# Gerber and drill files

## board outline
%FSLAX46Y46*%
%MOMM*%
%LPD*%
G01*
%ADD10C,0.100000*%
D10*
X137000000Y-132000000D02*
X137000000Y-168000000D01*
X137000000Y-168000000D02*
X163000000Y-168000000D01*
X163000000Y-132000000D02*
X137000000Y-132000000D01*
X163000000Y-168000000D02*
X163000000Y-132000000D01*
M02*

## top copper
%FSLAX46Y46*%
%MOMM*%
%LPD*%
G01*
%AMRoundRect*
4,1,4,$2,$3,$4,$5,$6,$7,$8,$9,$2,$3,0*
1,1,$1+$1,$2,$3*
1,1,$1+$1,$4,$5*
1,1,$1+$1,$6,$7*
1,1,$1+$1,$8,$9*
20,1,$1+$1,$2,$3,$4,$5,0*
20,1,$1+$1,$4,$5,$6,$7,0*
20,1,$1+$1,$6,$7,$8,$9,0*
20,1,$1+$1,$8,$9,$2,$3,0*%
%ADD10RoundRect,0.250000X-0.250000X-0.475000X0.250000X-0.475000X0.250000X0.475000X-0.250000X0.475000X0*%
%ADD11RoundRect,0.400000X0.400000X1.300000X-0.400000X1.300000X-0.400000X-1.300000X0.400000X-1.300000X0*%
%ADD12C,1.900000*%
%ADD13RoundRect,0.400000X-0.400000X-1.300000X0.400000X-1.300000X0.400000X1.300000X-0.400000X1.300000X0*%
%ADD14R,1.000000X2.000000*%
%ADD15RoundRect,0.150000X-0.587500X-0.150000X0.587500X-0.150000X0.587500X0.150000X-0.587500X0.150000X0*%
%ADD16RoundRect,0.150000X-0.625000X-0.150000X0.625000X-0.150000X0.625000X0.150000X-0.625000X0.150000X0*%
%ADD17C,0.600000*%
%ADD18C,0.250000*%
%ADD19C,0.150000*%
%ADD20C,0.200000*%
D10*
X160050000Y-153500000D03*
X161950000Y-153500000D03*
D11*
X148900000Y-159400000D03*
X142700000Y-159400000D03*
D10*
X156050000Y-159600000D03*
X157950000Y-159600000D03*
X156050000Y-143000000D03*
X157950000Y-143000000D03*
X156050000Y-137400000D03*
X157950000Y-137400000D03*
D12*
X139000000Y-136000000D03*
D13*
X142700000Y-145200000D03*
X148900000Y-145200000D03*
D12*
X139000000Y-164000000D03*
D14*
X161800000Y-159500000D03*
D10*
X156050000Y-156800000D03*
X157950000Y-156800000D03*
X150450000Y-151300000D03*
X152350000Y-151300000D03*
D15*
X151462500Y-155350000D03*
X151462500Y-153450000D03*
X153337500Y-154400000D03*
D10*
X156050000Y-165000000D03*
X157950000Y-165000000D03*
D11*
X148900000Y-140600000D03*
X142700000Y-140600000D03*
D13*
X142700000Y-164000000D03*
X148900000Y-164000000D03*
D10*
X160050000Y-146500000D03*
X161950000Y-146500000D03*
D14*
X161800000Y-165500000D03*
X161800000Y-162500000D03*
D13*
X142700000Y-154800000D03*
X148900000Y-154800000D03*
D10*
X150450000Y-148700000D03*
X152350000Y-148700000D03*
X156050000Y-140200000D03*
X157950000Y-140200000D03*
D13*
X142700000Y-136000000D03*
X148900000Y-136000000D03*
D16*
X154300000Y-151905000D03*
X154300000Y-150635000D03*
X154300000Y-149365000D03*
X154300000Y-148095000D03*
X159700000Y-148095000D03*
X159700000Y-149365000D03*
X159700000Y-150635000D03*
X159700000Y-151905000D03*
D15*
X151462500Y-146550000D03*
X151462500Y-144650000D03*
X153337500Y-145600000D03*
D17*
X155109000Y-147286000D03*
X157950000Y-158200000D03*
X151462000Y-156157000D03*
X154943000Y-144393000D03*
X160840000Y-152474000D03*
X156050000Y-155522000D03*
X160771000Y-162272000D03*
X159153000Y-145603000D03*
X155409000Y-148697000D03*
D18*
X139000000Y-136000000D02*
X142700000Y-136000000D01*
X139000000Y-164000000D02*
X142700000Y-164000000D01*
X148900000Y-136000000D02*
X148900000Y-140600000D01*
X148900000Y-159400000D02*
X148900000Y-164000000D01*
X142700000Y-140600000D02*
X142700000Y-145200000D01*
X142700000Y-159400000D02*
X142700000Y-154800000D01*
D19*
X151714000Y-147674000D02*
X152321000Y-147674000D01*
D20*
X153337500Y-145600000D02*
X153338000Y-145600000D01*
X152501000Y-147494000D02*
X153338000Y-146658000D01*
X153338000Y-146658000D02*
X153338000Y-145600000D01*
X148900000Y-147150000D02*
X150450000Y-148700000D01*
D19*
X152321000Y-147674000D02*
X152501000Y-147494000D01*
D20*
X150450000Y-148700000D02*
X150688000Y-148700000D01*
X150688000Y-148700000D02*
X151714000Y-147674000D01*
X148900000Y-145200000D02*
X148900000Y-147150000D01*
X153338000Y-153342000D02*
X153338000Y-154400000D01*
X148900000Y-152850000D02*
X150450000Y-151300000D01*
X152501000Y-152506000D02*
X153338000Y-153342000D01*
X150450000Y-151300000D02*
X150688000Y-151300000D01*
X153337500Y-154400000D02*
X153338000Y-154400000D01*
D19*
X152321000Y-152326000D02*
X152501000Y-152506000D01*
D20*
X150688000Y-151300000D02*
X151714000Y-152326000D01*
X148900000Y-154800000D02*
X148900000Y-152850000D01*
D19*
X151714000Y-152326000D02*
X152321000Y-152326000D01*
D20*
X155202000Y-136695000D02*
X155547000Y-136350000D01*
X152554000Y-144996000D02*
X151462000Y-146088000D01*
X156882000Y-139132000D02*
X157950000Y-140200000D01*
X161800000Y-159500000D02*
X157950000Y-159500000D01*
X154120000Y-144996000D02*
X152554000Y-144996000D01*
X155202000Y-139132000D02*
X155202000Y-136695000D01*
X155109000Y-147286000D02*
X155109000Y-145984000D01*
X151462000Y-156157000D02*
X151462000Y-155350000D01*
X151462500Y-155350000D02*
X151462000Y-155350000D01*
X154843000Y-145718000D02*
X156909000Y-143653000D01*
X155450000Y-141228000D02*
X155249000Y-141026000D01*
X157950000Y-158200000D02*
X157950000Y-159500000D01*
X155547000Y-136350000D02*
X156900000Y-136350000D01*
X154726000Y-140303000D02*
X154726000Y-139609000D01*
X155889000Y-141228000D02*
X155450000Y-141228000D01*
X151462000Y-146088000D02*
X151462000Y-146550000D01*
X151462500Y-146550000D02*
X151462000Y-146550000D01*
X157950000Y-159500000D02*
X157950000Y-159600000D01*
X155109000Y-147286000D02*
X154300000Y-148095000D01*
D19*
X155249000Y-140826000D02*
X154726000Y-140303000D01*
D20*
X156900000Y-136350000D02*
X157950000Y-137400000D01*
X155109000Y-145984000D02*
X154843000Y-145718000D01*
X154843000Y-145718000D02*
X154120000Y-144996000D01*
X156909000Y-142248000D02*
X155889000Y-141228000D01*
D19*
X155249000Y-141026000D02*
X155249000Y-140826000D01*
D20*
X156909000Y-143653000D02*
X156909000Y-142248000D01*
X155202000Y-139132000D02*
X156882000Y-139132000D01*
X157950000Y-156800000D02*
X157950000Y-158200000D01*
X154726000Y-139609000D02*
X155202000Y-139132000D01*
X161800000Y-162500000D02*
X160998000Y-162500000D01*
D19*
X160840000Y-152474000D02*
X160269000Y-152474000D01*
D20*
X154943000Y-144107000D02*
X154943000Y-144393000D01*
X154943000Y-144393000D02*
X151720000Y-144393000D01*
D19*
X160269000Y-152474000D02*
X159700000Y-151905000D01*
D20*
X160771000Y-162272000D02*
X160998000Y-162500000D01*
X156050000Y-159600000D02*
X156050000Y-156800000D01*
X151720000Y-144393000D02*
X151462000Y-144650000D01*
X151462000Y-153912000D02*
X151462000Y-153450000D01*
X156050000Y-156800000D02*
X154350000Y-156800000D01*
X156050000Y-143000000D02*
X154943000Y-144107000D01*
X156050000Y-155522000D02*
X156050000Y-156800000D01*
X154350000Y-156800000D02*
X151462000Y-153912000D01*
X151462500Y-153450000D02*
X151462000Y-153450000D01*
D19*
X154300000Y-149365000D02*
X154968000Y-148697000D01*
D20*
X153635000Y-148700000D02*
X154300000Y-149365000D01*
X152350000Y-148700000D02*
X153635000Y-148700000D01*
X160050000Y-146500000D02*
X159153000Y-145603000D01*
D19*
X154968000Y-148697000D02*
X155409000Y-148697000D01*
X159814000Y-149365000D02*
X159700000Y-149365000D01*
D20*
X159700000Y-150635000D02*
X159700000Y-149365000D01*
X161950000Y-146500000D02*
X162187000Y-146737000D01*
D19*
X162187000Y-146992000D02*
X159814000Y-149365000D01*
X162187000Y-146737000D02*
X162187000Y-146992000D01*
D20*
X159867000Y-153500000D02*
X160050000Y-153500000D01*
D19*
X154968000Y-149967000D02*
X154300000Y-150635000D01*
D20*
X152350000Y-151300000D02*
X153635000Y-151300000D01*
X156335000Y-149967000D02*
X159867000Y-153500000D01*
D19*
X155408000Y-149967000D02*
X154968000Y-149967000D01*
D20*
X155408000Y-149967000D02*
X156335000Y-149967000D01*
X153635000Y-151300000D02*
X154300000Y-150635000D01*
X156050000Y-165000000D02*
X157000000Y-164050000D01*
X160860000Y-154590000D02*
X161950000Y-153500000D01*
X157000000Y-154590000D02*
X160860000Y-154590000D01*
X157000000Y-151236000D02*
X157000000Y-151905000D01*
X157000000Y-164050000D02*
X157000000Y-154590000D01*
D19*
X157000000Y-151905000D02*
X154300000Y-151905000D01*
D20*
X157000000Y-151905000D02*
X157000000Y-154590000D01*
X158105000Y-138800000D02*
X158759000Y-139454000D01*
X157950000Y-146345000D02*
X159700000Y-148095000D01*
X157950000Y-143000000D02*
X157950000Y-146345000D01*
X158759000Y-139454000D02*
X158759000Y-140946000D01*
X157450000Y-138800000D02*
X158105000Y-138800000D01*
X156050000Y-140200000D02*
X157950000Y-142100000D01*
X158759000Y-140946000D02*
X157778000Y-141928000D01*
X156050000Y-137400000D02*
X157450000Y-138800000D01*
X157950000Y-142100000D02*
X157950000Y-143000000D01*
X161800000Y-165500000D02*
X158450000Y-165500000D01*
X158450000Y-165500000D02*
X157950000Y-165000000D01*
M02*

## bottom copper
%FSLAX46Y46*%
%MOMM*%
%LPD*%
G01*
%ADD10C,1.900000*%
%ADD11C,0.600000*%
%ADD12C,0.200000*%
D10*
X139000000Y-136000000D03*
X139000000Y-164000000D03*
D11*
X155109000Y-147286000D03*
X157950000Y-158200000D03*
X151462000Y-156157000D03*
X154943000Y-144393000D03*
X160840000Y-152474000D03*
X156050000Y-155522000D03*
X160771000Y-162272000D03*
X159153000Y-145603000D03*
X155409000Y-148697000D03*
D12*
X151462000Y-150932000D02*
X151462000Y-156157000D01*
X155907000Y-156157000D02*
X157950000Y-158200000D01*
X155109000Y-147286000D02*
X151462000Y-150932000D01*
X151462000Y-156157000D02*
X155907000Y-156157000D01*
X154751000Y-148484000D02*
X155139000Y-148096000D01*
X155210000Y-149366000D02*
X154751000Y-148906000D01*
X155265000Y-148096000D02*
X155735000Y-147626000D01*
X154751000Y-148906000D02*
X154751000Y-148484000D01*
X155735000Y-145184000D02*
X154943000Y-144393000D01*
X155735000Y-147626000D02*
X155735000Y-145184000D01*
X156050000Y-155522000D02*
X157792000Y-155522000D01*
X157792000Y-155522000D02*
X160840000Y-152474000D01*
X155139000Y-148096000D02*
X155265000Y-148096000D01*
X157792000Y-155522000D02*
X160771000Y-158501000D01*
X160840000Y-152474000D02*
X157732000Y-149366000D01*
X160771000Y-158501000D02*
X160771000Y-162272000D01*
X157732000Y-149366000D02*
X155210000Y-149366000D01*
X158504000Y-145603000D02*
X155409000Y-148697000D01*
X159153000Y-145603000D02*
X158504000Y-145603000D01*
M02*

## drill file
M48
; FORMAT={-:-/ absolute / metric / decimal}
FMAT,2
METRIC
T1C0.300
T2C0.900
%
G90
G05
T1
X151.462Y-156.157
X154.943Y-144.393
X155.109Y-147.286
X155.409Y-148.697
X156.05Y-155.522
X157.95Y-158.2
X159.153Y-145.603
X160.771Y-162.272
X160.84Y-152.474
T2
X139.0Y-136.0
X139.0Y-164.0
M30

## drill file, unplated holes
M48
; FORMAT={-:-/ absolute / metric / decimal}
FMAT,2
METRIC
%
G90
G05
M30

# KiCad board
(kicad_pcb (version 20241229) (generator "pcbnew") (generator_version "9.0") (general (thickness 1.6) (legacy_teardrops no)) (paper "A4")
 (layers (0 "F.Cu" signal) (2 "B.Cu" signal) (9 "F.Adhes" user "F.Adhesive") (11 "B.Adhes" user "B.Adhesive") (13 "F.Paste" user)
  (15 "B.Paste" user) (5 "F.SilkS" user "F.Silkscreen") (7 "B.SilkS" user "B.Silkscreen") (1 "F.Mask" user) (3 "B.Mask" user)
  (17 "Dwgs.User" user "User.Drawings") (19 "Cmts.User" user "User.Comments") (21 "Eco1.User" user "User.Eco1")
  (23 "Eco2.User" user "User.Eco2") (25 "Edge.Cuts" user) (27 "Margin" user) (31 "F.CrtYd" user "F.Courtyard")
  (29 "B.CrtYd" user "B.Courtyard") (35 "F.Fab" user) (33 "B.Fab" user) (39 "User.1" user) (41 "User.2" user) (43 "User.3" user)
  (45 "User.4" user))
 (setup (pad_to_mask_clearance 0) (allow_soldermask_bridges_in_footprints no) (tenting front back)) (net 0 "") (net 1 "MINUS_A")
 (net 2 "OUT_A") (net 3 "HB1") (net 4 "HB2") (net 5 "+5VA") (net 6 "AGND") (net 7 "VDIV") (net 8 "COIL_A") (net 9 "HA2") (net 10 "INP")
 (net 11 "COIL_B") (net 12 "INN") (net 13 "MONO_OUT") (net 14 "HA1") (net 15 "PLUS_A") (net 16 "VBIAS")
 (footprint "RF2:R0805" (layer "F.Cu") (at 161 153.5)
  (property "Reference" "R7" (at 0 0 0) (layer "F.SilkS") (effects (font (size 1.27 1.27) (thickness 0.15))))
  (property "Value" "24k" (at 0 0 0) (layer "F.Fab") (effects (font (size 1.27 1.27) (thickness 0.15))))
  (pad "1" smd roundrect (at -0.95 0) (size 1 1.45) (layers "F.Cu" "F.Mask" "F.Paste") (roundrect_rratio 0.25) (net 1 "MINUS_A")
   (thermal_bridge_angle 45))
  (pad "2" smd roundrect (at 0.95 0) (size 1 1.45) (layers "F.Cu" "F.Mask" "F.Paste") (roundrect_rratio 0.25) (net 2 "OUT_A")
   (thermal_bridge_angle 45)))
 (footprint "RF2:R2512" (layer "F.Cu") (at 145.8 159.4 180)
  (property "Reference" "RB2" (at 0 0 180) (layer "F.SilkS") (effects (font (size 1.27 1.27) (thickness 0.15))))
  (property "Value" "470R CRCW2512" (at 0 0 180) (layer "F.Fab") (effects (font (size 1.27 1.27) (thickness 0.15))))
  (pad "1" smd roundrect (at -3.1 0 180) (size 1.6 3.4) (layers "F.Cu" "F.Mask" "F.Paste") (roundrect_rratio 0.25) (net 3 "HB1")
   (thermal_bridge_angle 45))
  (pad "2" smd roundrect (at 3.1 0 180) (size 1.6 3.4) (layers "F.Cu" "F.Mask" "F.Paste") (roundrect_rratio 0.25) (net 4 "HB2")
   (thermal_bridge_angle 45)))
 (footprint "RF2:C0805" (layer "F.Cu") (at 157 159.6)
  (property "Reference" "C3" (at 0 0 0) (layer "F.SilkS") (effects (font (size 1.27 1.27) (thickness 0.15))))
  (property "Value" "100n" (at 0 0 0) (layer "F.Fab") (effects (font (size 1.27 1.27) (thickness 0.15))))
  (pad "1" smd roundrect (at -0.95 0) (size 1 1.45) (layers "F.Cu" "F.Mask" "F.Paste") (roundrect_rratio 0.25) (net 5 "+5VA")
   (thermal_bridge_angle 45))
  (pad "2" smd roundrect (at 0.95 0) (size 1 1.45) (layers "F.Cu" "F.Mask" "F.Paste") (roundrect_rratio 0.25) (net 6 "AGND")
   (thermal_bridge_angle 45)))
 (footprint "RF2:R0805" (layer "F.Cu") (at 157 143)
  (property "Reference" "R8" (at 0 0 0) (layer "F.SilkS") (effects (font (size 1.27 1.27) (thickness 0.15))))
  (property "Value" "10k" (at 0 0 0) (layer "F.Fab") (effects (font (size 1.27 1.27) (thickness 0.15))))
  (pad "1" smd roundrect (at -0.95 0) (size 1 1.45) (layers "F.Cu" "F.Mask" "F.Paste") (roundrect_rratio 0.25) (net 5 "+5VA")
   (thermal_bridge_angle 45))
  (pad "2" smd roundrect (at 0.95 0) (size 1 1.45) (layers "F.Cu" "F.Mask" "F.Paste") (roundrect_rratio 0.25) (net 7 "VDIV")
   (thermal_bridge_angle 45)))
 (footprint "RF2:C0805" (layer "F.Cu") (at 157 137.4)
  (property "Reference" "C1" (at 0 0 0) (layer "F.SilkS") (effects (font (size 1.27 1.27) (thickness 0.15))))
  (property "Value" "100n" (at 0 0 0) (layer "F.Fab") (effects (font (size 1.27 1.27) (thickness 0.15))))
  (pad "1" smd roundrect (at -0.95 0) (size 1 1.45) (layers "F.Cu" "F.Mask" "F.Paste") (roundrect_rratio 0.25) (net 7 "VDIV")
   (thermal_bridge_angle 45))
  (pad "2" smd roundrect (at 0.95 0) (size 1 1.45) (layers "F.Cu" "F.Mask" "F.Paste") (roundrect_rratio 0.25) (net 6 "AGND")
   (thermal_bridge_angle 45)))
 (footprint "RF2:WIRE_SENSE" (layer "F.Cu") (at 139 136)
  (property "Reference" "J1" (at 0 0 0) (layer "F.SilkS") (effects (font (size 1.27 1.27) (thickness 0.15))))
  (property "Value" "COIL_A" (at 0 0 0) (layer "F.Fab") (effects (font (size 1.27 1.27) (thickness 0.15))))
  (pad "1" thru_hole circle (at 0 0) (size 1.9 1.9) (drill 0.9) (layers "*.Cu" "*.Mask") (remove_unused_layers no) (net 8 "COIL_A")))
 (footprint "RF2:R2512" (layer "F.Cu") (at 145.8 145.2)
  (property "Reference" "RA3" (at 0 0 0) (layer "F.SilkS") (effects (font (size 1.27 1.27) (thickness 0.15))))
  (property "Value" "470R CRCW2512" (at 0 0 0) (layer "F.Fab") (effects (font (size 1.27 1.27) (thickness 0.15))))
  (pad "1" smd roundrect (at -3.1 0) (size 1.6 3.4) (layers "F.Cu" "F.Mask" "F.Paste") (roundrect_rratio 0.25) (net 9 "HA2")
   (thermal_bridge_angle 45))
  (pad "2" smd roundrect (at 3.1 0) (size 1.6 3.4) (layers "F.Cu" "F.Mask" "F.Paste") (roundrect_rratio 0.25) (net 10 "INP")
   (thermal_bridge_angle 45)))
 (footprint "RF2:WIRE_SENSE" (layer "F.Cu") (at 139 164)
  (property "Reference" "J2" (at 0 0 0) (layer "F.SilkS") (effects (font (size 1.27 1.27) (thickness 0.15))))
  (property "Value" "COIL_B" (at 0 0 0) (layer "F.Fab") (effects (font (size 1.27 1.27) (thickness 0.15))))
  (pad "1" thru_hole circle (at 0 0) (size 1.9 1.9) (drill 0.9) (layers "*.Cu" "*.Mask") (remove_unused_layers no) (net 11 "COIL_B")))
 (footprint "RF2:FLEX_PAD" (layer "F.Cu") (at 161.8 159.5)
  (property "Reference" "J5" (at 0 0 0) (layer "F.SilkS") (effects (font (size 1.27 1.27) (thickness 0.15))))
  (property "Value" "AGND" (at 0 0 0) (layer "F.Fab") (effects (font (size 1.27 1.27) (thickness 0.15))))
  (pad "1" smd rect (at 0 0) (size 1 2) (layers "F.Cu" "F.Mask" "F.Paste") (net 6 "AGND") (thermal_bridge_angle 45)))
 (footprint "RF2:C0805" (layer "F.Cu") (at 157 156.8)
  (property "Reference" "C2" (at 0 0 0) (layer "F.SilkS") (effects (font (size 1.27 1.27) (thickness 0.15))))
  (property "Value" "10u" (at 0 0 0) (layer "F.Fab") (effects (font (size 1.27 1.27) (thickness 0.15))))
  (pad "1" smd roundrect (at -0.95 0) (size 1 1.45) (layers "F.Cu" "F.Mask" "F.Paste") (roundrect_rratio 0.25) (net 5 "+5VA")
   (thermal_bridge_angle 45))
  (pad "2" smd roundrect (at 0.95 0) (size 1 1.45) (layers "F.Cu" "F.Mask" "F.Paste") (roundrect_rratio 0.25) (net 6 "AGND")
   (thermal_bridge_angle 45)))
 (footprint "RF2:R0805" (layer "F.Cu") (at 151.4 151.3)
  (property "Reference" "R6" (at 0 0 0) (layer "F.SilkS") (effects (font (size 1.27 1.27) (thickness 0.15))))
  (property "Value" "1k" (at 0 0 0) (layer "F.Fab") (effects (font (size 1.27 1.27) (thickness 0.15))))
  (pad "1" smd roundrect (at -0.95 0) (size 1 1.45) (layers "F.Cu" "F.Mask" "F.Paste") (roundrect_rratio 0.25) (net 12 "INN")
   (thermal_bridge_angle 45))
  (pad "2" smd roundrect (at 0.95 0) (size 1 1.45) (layers "F.Cu" "F.Mask" "F.Paste") (roundrect_rratio 0.25) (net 1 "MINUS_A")
   (thermal_bridge_angle 45)))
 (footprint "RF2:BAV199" (layer "F.Cu") (at 152.4 154.4)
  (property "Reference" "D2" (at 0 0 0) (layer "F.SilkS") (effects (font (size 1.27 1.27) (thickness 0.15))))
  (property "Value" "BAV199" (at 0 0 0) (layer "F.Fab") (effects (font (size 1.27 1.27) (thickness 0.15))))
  (pad "1" smd roundrect (at -0.9375 0.95) (size 1.475 0.6) (layers "F.Cu" "F.Mask" "F.Paste") (roundrect_rratio 0.25) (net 6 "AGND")
   (thermal_bridge_angle 45))
  (pad "2" smd roundrect (at -0.9375 -0.95) (size 1.475 0.6) (layers "F.Cu" "F.Mask" "F.Paste") (roundrect_rratio 0.25) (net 5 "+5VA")
   (thermal_bridge_angle 45))
  (pad "3" smd roundrect (at 0.9375 0) (size 1.475 0.6) (layers "F.Cu" "F.Mask" "F.Paste") (roundrect_rratio 0.25) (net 12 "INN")
   (thermal_bridge_angle 45)))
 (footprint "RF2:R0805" (layer "F.Cu") (at 157 165)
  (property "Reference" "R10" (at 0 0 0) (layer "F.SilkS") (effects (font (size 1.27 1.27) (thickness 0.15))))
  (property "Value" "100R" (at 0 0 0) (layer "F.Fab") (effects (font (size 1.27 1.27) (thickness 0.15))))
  (pad "1" smd roundrect (at -0.95 0) (size 1 1.45) (layers "F.Cu" "F.Mask" "F.Paste") (roundrect_rratio 0.25) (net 2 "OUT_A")
   (thermal_bridge_angle 45))
  (pad "2" smd roundrect (at 0.95 0) (size 1 1.45) (layers "F.Cu" "F.Mask" "F.Paste") (roundrect_rratio 0.25) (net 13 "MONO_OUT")
   (thermal_bridge_angle 45)))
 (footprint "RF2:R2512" (layer "F.Cu") (at 145.8 140.6 180)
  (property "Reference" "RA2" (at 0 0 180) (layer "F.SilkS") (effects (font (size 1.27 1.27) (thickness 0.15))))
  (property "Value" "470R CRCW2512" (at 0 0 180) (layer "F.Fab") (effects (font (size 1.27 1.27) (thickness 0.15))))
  (pad "1" smd roundrect (at -3.1 0 180) (size 1.6 3.4) (layers "F.Cu" "F.Mask" "F.Paste") (roundrect_rratio 0.25) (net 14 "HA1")
   (thermal_bridge_angle 45))
  (pad "2" smd roundrect (at 3.1 0 180) (size 1.6 3.4) (layers "F.Cu" "F.Mask" "F.Paste") (roundrect_rratio 0.25) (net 9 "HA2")
   (thermal_bridge_angle 45)))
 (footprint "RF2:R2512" (layer "F.Cu") (at 145.8 164)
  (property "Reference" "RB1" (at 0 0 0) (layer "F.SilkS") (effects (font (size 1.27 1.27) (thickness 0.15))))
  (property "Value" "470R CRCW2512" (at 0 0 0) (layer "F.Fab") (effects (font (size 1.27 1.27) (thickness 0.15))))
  (pad "1" smd roundrect (at -3.1 0) (size 1.6 3.4) (layers "F.Cu" "F.Mask" "F.Paste") (roundrect_rratio 0.25) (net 11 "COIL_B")
   (thermal_bridge_angle 45))
  (pad "2" smd roundrect (at 3.1 0) (size 1.6 3.4) (layers "F.Cu" "F.Mask" "F.Paste") (roundrect_rratio 0.25) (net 3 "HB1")
   (thermal_bridge_angle 45)))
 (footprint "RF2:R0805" (layer "F.Cu") (at 161 146.5)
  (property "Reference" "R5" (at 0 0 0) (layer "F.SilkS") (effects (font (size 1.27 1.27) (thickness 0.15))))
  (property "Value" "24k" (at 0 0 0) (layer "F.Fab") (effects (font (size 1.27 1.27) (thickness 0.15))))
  (pad "1" smd roundrect (at -0.95 0) (size 1 1.45) (layers "F.Cu" "F.Mask" "F.Paste") (roundrect_rratio 0.25) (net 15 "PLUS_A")
   (thermal_bridge_angle 45))
  (pad "2" smd roundrect (at 0.95 0) (size 1 1.45) (layers "F.Cu" "F.Mask" "F.Paste") (roundrect_rratio 0.25) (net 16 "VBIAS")
   (thermal_bridge_angle 45)))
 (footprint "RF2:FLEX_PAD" (layer "F.Cu") (at 161.8 165.5)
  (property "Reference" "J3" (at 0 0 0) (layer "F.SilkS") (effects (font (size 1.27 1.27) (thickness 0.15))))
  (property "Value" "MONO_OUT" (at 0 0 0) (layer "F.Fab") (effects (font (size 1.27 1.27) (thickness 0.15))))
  (pad "1" smd rect (at 0 0) (size 1 2) (layers "F.Cu" "F.Mask" "F.Paste") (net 13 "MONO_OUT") (thermal_bridge_angle 45)))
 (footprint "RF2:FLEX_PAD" (layer "F.Cu") (at 161.8 162.5)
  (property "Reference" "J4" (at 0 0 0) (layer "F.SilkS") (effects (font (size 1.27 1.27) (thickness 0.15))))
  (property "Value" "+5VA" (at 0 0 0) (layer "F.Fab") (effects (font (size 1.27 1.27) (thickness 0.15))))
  (pad "1" smd rect (at 0 0) (size 1 2) (layers "F.Cu" "F.Mask" "F.Paste") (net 5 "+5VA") (thermal_bridge_angle 45)))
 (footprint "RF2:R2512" (layer "F.Cu") (at 145.8 154.8)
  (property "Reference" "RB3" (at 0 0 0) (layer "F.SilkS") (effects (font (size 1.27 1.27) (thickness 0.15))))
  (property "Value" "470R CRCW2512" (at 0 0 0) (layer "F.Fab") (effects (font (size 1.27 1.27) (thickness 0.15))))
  (pad "1" smd roundrect (at -3.1 0) (size 1.6 3.4) (layers "F.Cu" "F.Mask" "F.Paste") (roundrect_rratio 0.25) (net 4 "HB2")
   (thermal_bridge_angle 45))
  (pad "2" smd roundrect (at 3.1 0) (size 1.6 3.4) (layers "F.Cu" "F.Mask" "F.Paste") (roundrect_rratio 0.25) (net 12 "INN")
   (thermal_bridge_angle 45)))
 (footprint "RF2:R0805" (layer "F.Cu") (at 151.4 148.7)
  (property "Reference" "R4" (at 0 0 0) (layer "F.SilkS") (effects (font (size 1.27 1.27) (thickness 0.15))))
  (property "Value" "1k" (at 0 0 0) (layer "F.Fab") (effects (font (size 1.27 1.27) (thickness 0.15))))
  (pad "1" smd roundrect (at -0.95 0) (size 1 1.45) (layers "F.Cu" "F.Mask" "F.Paste") (roundrect_rratio 0.25) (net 10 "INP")
   (thermal_bridge_angle 45))
  (pad "2" smd roundrect (at 0.95 0) (size 1 1.45) (layers "F.Cu" "F.Mask" "F.Paste") (roundrect_rratio 0.25) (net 15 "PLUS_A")
   (thermal_bridge_angle 45)))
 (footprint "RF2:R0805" (layer "F.Cu") (at 157 140.2)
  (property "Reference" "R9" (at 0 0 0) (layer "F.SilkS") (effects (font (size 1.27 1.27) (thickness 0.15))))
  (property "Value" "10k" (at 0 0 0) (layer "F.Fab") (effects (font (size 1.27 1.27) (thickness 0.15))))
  (pad "1" smd roundrect (at -0.95 0) (size 1 1.45) (layers "F.Cu" "F.Mask" "F.Paste") (roundrect_rratio 0.25) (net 7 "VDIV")
   (thermal_bridge_angle 45))
  (pad "2" smd roundrect (at 0.95 0) (size 1 1.45) (layers "F.Cu" "F.Mask" "F.Paste") (roundrect_rratio 0.25) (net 6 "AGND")
   (thermal_bridge_angle 45)))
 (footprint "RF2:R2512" (layer "F.Cu") (at 145.8 136)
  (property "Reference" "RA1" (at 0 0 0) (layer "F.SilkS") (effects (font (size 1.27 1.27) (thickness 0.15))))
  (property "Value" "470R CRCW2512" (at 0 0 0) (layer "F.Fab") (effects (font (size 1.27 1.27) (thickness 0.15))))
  (pad "1" smd roundrect (at -3.1 0) (size 1.6 3.4) (layers "F.Cu" "F.Mask" "F.Paste") (roundrect_rratio 0.25) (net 8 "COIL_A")
   (thermal_bridge_angle 45))
  (pad "2" smd roundrect (at 3.1 0) (size 1.6 3.4) (layers "F.Cu" "F.Mask" "F.Paste") (roundrect_rratio 0.25) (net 14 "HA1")
   (thermal_bridge_angle 45)))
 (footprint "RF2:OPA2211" (layer "F.Cu") (at 157 150)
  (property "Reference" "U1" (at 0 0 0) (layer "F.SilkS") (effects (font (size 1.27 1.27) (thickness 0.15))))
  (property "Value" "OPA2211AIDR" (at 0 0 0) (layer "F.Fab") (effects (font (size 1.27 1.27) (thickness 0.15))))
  (pad "1" smd roundrect (at -2.7 1.905) (size 1.55 0.6) (layers "F.Cu" "F.Mask" "F.Paste") (roundrect_rratio 0.25) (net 2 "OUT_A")
   (thermal_bridge_angle 45))
  (pad "2" smd roundrect (at -2.7 0.635) (size 1.55 0.6) (layers "F.Cu" "F.Mask" "F.Paste") (roundrect_rratio 0.25) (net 1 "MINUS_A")
   (thermal_bridge_angle 45))
  (pad "3" smd roundrect (at -2.7 -0.635) (size 1.55 0.6) (layers "F.Cu" "F.Mask" "F.Paste") (roundrect_rratio 0.25) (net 15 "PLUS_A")
   (thermal_bridge_angle 45))
  (pad "4" smd roundrect (at -2.7 -1.905) (size 1.55 0.6) (layers "F.Cu" "F.Mask" "F.Paste") (roundrect_rratio 0.25) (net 6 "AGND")
   (thermal_bridge_angle 45))
  (pad "5" smd roundrect (at 2.7 -1.905) (size 1.55 0.6) (layers "F.Cu" "F.Mask" "F.Paste") (roundrect_rratio 0.25) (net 7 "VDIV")
   (thermal_bridge_angle 45))
  (pad "6" smd roundrect (at 2.7 -0.635) (size 1.55 0.6) (layers "F.Cu" "F.Mask" "F.Paste") (roundrect_rratio 0.25) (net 16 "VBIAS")
   (thermal_bridge_angle 45))
  (pad "7" smd roundrect (at 2.7 0.635) (size 1.55 0.6) (layers "F.Cu" "F.Mask" "F.Paste") (roundrect_rratio 0.25) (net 16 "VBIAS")
   (thermal_bridge_angle 45))
  (pad "8" smd roundrect (at 2.7 1.905) (size 1.55 0.6) (layers "F.Cu" "F.Mask" "F.Paste") (roundrect_rratio 0.25) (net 5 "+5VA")
   (thermal_bridge_angle 45)))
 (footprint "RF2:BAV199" (layer "F.Cu") (at 152.4 145.6)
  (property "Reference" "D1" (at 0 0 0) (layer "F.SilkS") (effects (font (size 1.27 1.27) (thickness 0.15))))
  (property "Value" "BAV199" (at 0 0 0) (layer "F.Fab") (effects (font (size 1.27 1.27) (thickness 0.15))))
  (pad "1" smd roundrect (at -0.9375 0.95) (size 1.475 0.6) (layers "F.Cu" "F.Mask" "F.Paste") (roundrect_rratio 0.25) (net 6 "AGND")
   (thermal_bridge_angle 45))
  (pad "2" smd roundrect (at -0.9375 -0.95) (size 1.475 0.6) (layers "F.Cu" "F.Mask" "F.Paste") (roundrect_rratio 0.25) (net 5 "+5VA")
   (thermal_bridge_angle 45))
  (pad "3" smd roundrect (at 0.9375 0) (size 1.475 0.6) (layers "F.Cu" "F.Mask" "F.Paste") (roundrect_rratio 0.25) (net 10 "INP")
   (thermal_bridge_angle 45)))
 (gr_line (start 137 132) (end 137 168) (stroke (width 0.1) (type default)) (layer "Edge.Cuts"))
 (gr_line (start 137 168) (end 163 168) (stroke (width 0.1) (type default)) (layer "Edge.Cuts"))
 (gr_line (start 163 132) (end 137 132) (stroke (width 0.1) (type default)) (layer "Edge.Cuts"))
 (gr_line (start 163 168) (end 163 132) (stroke (width 0.1) (type default)) (layer "Edge.Cuts"))
 (segment (start 139 136) (end 142.7 136) (width 0.25) (layer "F.Cu") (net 8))
 (segment (start 139 164) (end 142.7 164) (width 0.25) (layer "F.Cu") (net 11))
 (segment (start 148.9 136) (end 148.9 140.6) (width 0.25) (layer "F.Cu") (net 14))
 (segment (start 148.9 159.4) (end 148.9 164) (width 0.25) (layer "F.Cu") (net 3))
 (segment (start 142.7 140.6) (end 142.7 145.2) (width 0.25) (layer "F.Cu") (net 9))
 (segment (start 142.7 159.4) (end 142.7 154.8) (width 0.25) (layer "F.Cu") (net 4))
 (segment (start 151.714 147.674) (end 152.321 147.674) (width 0.15) (layer "F.Cu") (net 10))
 (segment (start 153.3375 145.6) (end 153.338 145.6) (width 0.2) (layer "F.Cu") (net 10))
 (segment (start 152.501 147.494) (end 153.338 146.658) (width 0.2) (layer "F.Cu") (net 10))
 (segment (start 153.338 146.658) (end 153.338 145.6) (width 0.2) (layer "F.Cu") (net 10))
 (segment (start 148.9 147.15) (end 150.45 148.7) (width 0.2) (layer "F.Cu") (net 10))
 (segment (start 152.321 147.674) (end 152.501 147.494) (width 0.15) (layer "F.Cu") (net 10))
 (segment (start 150.45 148.7) (end 150.688 148.7) (width 0.2) (layer "F.Cu") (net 10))
 (segment (start 150.688 148.7) (end 151.714 147.674) (width 0.2) (layer "F.Cu") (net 10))
 (segment (start 148.9 145.2) (end 148.9 147.15) (width 0.2) (layer "F.Cu") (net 10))
 (segment (start 153.338 153.342) (end 153.338 154.4) (width 0.2) (layer "F.Cu") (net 12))
 (segment (start 148.9 152.85) (end 150.45 151.3) (width 0.2) (layer "F.Cu") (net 12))
 (segment (start 152.501 152.506) (end 153.338 153.342) (width 0.2) (layer "F.Cu") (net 12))
 (segment (start 150.45 151.3) (end 150.688 151.3) (width 0.2) (layer "F.Cu") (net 12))
 (segment (start 153.3375 154.4) (end 153.338 154.4) (width 0.2) (layer "F.Cu") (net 12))
 (segment (start 152.321 152.326) (end 152.501 152.506) (width 0.15) (layer "F.Cu") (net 12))
 (segment (start 150.688 151.3) (end 151.714 152.326) (width 0.2) (layer "F.Cu") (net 12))
 (segment (start 148.9 154.8) (end 148.9 152.85) (width 0.2) (layer "F.Cu") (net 12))
 (segment (start 151.714 152.326) (end 152.321 152.326) (width 0.15) (layer "F.Cu") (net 12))
 (segment (start 155.202 136.695) (end 155.547 136.35) (width 0.2) (layer "F.Cu") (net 6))
 (segment (start 152.554 144.996) (end 151.462 146.088) (width 0.2) (layer "F.Cu") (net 6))
 (segment (start 156.882 139.132) (end 157.95 140.2) (width 0.2) (layer "F.Cu") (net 6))
 (segment (start 161.8 159.5) (end 157.95 159.5) (width 0.2) (layer "F.Cu") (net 6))
 (segment (start 154.12 144.996) (end 152.554 144.996) (width 0.2) (layer "F.Cu") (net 6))
 (segment (start 155.202 139.132) (end 155.202 136.695) (width 0.2) (layer "F.Cu") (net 6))
 (segment (start 155.109 147.286) (end 155.109 145.984) (width 0.2) (layer "F.Cu") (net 6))
 (segment (start 151.462 156.157) (end 151.462 155.35) (width 0.2) (layer "F.Cu") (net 6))
 (segment (start 151.4625 155.35) (end 151.462 155.35) (width 0.2) (layer "F.Cu") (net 6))
 (segment (start 154.843 145.718) (end 156.909 143.653) (width 0.2) (layer "F.Cu") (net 6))
 (segment (start 155.45 141.228) (end 155.249 141.026) (width 0.2) (layer "F.Cu") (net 6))
 (segment (start 157.95 158.2) (end 157.95 159.5) (width 0.2) (layer "F.Cu") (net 6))
 (segment (start 155.547 136.35) (end 156.9 136.35) (width 0.2) (layer "F.Cu") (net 6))
 (segment (start 154.726 140.303) (end 154.726 139.609) (width 0.2) (layer "F.Cu") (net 6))
 (segment (start 155.889 141.228) (end 155.45 141.228) (width 0.2) (layer "F.Cu") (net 6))
 (segment (start 151.462 146.088) (end 151.462 146.55) (width 0.2) (layer "F.Cu") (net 6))
 (segment (start 151.4625 146.55) (end 151.462 146.55) (width 0.2) (layer "F.Cu") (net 6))
 (segment (start 157.95 159.5) (end 157.95 159.6) (width 0.2) (layer "F.Cu") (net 6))
 (segment (start 155.109 147.286) (end 154.3 148.095) (width 0.2) (layer "F.Cu") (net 6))
 (segment (start 155.249 140.826) (end 154.726 140.303) (width 0.15) (layer "F.Cu") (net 6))
 (segment (start 156.9 136.35) (end 157.95 137.4) (width 0.2) (layer "F.Cu") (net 6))
 (segment (start 155.109 145.984) (end 154.843 145.718) (width 0.2) (layer "F.Cu") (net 6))
 (segment (start 154.843 145.718) (end 154.12 144.996) (width 0.2) (layer "F.Cu") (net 6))
 (segment (start 156.909 142.248) (end 155.889 141.228) (width 0.2) (layer "F.Cu") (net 6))
 (segment (start 155.249 141.026) (end 155.249 140.826) (width 0.15) (layer "F.Cu") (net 6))
 (segment (start 156.909 143.653) (end 156.909 142.248) (width 0.2) (layer "F.Cu") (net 6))
 (segment (start 155.202 139.132) (end 156.882 139.132) (width 0.2) (layer "F.Cu") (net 6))
 (segment (start 157.95 156.8) (end 157.95 158.2) (width 0.2) (layer "F.Cu") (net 6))
 (segment (start 154.726 139.609) (end 155.202 139.132) (width 0.2) (layer "F.Cu") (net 6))
 (via (at 155.109 147.286) (size 0.6) (drill 0.3) (layers "F.Cu" "B.Cu") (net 6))
 (via (at 157.95 158.2) (size 0.6) (drill 0.3) (layers "F.Cu" "B.Cu") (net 6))
 (via (at 151.462 156.157) (size 0.6) (drill 0.3) (layers "F.Cu" "B.Cu") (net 6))
 (segment (start 151.462 150.932) (end 151.462 156.157) (width 0.2) (layer "B.Cu") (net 6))
 (segment (start 155.907 156.157) (end 157.95 158.2) (width 0.2) (layer "B.Cu") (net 6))
 (segment (start 155.109 147.286) (end 151.462 150.932) (width 0.2) (layer "B.Cu") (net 6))
 (segment (start 151.462 156.157) (end 155.907 156.157) (width 0.2) (layer "B.Cu") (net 6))
 (segment (start 161.8 162.5) (end 160.998 162.5) (width 0.2) (layer "F.Cu") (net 5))
 (segment (start 160.84 152.474) (end 160.269 152.474) (width 0.15) (layer "F.Cu") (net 5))
 (segment (start 154.943 144.107) (end 154.943 144.393) (width 0.2) (layer "F.Cu") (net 5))
 (segment (start 154.943 144.393) (end 151.72 144.393) (width 0.2) (layer "F.Cu") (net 5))
 (segment (start 160.269 152.474) (end 159.7 151.905) (width 0.15) (layer "F.Cu") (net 5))
 (segment (start 160.771 162.272) (end 160.998 162.5) (width 0.2) (layer "F.Cu") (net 5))
 (segment (start 156.05 159.6) (end 156.05 156.8) (width 0.2) (layer "F.Cu") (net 5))
 (segment (start 151.72 144.393) (end 151.462 144.65) (width 0.2) (layer "F.Cu") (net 5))
 (segment (start 151.462 153.912) (end 151.462 153.45) (width 0.2) (layer "F.Cu") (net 5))
 (segment (start 156.05 156.8) (end 154.35 156.8) (width 0.2) (layer "F.Cu") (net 5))
 (segment (start 156.05 143) (end 154.943 144.107) (width 0.2) (layer "F.Cu") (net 5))
 (segment (start 156.05 155.522) (end 156.05 156.8) (width 0.2) (layer "F.Cu") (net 5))
 (segment (start 154.35 156.8) (end 151.462 153.912) (width 0.2) (layer "F.Cu") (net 5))
 (segment (start 151.4625 153.45) (end 151.462 153.45) (width 0.2) (layer "F.Cu") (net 5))
 (via (at 154.943 144.393) (size 0.6) (drill 0.3) (layers "F.Cu" "B.Cu") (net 5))
 (via (at 160.84 152.474) (size 0.6) (drill 0.3) (layers "F.Cu" "B.Cu") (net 5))
 (via (at 156.05 155.522) (size 0.6) (drill 0.3) (layers "F.Cu" "B.Cu") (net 5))
 (via (at 160.771 162.272) (size 0.6) (drill 0.3) (layers "F.Cu" "B.Cu") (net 5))
 (segment (start 154.751 148.484) (end 155.139 148.096) (width 0.2) (layer "B.Cu") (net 5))
 (segment (start 155.21 149.366) (end 154.751 148.906) (width 0.2) (layer "B.Cu") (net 5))
 (segment (start 155.265 148.096) (end 155.735 147.626) (width 0.2) (layer "B.Cu") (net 5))
 (segment (start 154.751 148.906) (end 154.751 148.484) (width 0.2) (layer "B.Cu") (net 5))
 (segment (start 155.735 145.184) (end 154.943 144.393) (width 0.2) (layer "B.Cu") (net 5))
 (segment (start 155.735 147.626) (end 155.735 145.184) (width 0.2) (layer "B.Cu") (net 5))
 (segment (start 156.05 155.522) (end 157.792 155.522) (width 0.2) (layer "B.Cu") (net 5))
 (segment (start 157.792 155.522) (end 160.84 152.474) (width 0.2) (layer "B.Cu") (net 5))
 (segment (start 155.139 148.096) (end 155.265 148.096) (width 0.2) (layer "B.Cu") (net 5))
 (segment (start 157.792 155.522) (end 160.771 158.501) (width 0.2) (layer "B.Cu") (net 5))
 (segment (start 160.84 152.474) (end 157.732 149.366) (width 0.2) (layer "B.Cu") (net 5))
 (segment (start 160.771 158.501) (end 160.771 162.272) (width 0.2) (layer "B.Cu") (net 5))
 (segment (start 157.732 149.366) (end 155.21 149.366) (width 0.2) (layer "B.Cu") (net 5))
 (segment (start 154.3 149.365) (end 154.968 148.697) (width 0.15) (layer "F.Cu") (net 15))
 (segment (start 153.635 148.7) (end 154.3 149.365) (width 0.2) (layer "F.Cu") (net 15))
 (segment (start 152.35 148.7) (end 153.635 148.7) (width 0.2) (layer "F.Cu") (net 15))
 (segment (start 160.05 146.5) (end 159.153 145.603) (width 0.2) (layer "F.Cu") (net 15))
 (segment (start 154.968 148.697) (end 155.409 148.697) (width 0.15) (layer "F.Cu") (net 15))
 (via (at 159.153 145.603) (size 0.6) (drill 0.3) (layers "F.Cu" "B.Cu") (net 15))
 (via (at 155.409 148.697) (size 0.6) (drill 0.3) (layers "F.Cu" "B.Cu") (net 15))
 (segment (start 158.504 145.603) (end 155.409 148.697) (width 0.2) (layer "B.Cu") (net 15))
 (segment (start 159.153 145.603) (end 158.504 145.603) (width 0.2) (layer "B.Cu") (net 15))
 (segment (start 159.814 149.365) (end 159.7 149.365) (width 0.15) (layer "F.Cu") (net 16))
 (segment (start 159.7 150.635) (end 159.7 149.365) (width 0.2) (layer "F.Cu") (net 16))
 (segment (start 161.95 146.5) (end 162.187 146.737) (width 0.2) (layer "F.Cu") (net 16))
 (segment (start 162.187 146.992) (end 159.814 149.365) (width 0.15) (layer "F.Cu") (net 16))
 (segment (start 162.187 146.737) (end 162.187 146.992) (width 0.15) (layer "F.Cu") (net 16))
 (segment (start 159.867 153.5) (end 160.05 153.5) (width 0.2) (layer "F.Cu") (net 1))
 (segment (start 154.968 149.967) (end 154.3 150.635) (width 0.15) (layer "F.Cu") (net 1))
 (segment (start 152.35 151.3) (end 153.635 151.3) (width 0.2) (layer "F.Cu") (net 1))
 (segment (start 156.335 149.967) (end 159.867 153.5) (width 0.2) (layer "F.Cu") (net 1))
 (segment (start 155.408 149.967) (end 154.968 149.967) (width 0.15) (layer "F.Cu") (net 1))
 (segment (start 155.408 149.967) (end 156.335 149.967) (width 0.2) (layer "F.Cu") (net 1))
 (segment (start 153.635 151.3) (end 154.3 150.635) (width 0.2) (layer "F.Cu") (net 1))
 (segment (start 156.05 165) (end 157 164.05) (width 0.2) (layer "F.Cu") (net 2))
 (segment (start 160.86 154.59) (end 161.95 153.5) (width 0.2) (layer "F.Cu") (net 2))
 (segment (start 157 154.59) (end 160.86 154.59) (width 0.2) (layer "F.Cu") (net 2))
 (segment (start 157 151.236) (end 157 151.905) (width 0.2) (layer "F.Cu") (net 2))
 (segment (start 157 164.05) (end 157 154.59) (width 0.2) (layer "F.Cu") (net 2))
 (segment (start 157 151.905) (end 154.3 151.905) (width 0.15) (layer "F.Cu") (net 2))
 (segment (start 157 151.905) (end 157 154.59) (width 0.2) (layer "F.Cu") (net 2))
 (segment (start 158.105 138.8) (end 158.759 139.454) (width 0.2) (layer "F.Cu") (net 7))
 (segment (start 157.95 146.345) (end 159.7 148.095) (width 0.2) (layer "F.Cu") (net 7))
 (segment (start 157.95 143) (end 157.95 146.345) (width 0.2) (layer "F.Cu") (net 7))
 (segment (start 158.759 139.454) (end 158.759 140.946) (width 0.2) (layer "F.Cu") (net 7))
 (segment (start 157.45 138.8) (end 158.105 138.8) (width 0.2) (layer "F.Cu") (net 7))
 (segment (start 156.05 140.2) (end 157.95 142.1) (width 0.2) (layer "F.Cu") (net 7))
 (segment (start 158.759 140.946) (end 157.778 141.928) (width 0.2) (layer "F.Cu") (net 7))
 (segment (start 156.05 137.4) (end 157.45 138.8) (width 0.2) (layer "F.Cu") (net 7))
 (segment (start 157.95 142.1) (end 157.95 143) (width 0.2) (layer "F.Cu") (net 7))
 (segment (start 161.8 165.5) (end 158.45 165.5) (width 0.2) (layer "F.Cu") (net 13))
 (segment (start 158.45 165.5) (end 157.95 165) (width 0.2) (layer "F.Cu") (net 13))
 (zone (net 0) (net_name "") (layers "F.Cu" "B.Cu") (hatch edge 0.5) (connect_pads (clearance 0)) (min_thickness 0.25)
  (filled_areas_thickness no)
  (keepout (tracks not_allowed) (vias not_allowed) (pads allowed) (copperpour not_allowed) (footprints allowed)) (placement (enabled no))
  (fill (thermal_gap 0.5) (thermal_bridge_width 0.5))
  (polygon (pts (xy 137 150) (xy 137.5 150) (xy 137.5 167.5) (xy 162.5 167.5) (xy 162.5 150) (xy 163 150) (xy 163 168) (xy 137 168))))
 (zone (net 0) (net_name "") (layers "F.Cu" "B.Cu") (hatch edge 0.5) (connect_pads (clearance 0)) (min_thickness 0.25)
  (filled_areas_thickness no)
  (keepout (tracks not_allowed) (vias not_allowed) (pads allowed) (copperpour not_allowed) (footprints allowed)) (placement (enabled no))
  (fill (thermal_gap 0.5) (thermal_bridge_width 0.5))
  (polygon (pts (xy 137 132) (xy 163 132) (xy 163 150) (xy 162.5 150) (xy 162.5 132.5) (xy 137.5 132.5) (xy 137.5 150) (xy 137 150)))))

